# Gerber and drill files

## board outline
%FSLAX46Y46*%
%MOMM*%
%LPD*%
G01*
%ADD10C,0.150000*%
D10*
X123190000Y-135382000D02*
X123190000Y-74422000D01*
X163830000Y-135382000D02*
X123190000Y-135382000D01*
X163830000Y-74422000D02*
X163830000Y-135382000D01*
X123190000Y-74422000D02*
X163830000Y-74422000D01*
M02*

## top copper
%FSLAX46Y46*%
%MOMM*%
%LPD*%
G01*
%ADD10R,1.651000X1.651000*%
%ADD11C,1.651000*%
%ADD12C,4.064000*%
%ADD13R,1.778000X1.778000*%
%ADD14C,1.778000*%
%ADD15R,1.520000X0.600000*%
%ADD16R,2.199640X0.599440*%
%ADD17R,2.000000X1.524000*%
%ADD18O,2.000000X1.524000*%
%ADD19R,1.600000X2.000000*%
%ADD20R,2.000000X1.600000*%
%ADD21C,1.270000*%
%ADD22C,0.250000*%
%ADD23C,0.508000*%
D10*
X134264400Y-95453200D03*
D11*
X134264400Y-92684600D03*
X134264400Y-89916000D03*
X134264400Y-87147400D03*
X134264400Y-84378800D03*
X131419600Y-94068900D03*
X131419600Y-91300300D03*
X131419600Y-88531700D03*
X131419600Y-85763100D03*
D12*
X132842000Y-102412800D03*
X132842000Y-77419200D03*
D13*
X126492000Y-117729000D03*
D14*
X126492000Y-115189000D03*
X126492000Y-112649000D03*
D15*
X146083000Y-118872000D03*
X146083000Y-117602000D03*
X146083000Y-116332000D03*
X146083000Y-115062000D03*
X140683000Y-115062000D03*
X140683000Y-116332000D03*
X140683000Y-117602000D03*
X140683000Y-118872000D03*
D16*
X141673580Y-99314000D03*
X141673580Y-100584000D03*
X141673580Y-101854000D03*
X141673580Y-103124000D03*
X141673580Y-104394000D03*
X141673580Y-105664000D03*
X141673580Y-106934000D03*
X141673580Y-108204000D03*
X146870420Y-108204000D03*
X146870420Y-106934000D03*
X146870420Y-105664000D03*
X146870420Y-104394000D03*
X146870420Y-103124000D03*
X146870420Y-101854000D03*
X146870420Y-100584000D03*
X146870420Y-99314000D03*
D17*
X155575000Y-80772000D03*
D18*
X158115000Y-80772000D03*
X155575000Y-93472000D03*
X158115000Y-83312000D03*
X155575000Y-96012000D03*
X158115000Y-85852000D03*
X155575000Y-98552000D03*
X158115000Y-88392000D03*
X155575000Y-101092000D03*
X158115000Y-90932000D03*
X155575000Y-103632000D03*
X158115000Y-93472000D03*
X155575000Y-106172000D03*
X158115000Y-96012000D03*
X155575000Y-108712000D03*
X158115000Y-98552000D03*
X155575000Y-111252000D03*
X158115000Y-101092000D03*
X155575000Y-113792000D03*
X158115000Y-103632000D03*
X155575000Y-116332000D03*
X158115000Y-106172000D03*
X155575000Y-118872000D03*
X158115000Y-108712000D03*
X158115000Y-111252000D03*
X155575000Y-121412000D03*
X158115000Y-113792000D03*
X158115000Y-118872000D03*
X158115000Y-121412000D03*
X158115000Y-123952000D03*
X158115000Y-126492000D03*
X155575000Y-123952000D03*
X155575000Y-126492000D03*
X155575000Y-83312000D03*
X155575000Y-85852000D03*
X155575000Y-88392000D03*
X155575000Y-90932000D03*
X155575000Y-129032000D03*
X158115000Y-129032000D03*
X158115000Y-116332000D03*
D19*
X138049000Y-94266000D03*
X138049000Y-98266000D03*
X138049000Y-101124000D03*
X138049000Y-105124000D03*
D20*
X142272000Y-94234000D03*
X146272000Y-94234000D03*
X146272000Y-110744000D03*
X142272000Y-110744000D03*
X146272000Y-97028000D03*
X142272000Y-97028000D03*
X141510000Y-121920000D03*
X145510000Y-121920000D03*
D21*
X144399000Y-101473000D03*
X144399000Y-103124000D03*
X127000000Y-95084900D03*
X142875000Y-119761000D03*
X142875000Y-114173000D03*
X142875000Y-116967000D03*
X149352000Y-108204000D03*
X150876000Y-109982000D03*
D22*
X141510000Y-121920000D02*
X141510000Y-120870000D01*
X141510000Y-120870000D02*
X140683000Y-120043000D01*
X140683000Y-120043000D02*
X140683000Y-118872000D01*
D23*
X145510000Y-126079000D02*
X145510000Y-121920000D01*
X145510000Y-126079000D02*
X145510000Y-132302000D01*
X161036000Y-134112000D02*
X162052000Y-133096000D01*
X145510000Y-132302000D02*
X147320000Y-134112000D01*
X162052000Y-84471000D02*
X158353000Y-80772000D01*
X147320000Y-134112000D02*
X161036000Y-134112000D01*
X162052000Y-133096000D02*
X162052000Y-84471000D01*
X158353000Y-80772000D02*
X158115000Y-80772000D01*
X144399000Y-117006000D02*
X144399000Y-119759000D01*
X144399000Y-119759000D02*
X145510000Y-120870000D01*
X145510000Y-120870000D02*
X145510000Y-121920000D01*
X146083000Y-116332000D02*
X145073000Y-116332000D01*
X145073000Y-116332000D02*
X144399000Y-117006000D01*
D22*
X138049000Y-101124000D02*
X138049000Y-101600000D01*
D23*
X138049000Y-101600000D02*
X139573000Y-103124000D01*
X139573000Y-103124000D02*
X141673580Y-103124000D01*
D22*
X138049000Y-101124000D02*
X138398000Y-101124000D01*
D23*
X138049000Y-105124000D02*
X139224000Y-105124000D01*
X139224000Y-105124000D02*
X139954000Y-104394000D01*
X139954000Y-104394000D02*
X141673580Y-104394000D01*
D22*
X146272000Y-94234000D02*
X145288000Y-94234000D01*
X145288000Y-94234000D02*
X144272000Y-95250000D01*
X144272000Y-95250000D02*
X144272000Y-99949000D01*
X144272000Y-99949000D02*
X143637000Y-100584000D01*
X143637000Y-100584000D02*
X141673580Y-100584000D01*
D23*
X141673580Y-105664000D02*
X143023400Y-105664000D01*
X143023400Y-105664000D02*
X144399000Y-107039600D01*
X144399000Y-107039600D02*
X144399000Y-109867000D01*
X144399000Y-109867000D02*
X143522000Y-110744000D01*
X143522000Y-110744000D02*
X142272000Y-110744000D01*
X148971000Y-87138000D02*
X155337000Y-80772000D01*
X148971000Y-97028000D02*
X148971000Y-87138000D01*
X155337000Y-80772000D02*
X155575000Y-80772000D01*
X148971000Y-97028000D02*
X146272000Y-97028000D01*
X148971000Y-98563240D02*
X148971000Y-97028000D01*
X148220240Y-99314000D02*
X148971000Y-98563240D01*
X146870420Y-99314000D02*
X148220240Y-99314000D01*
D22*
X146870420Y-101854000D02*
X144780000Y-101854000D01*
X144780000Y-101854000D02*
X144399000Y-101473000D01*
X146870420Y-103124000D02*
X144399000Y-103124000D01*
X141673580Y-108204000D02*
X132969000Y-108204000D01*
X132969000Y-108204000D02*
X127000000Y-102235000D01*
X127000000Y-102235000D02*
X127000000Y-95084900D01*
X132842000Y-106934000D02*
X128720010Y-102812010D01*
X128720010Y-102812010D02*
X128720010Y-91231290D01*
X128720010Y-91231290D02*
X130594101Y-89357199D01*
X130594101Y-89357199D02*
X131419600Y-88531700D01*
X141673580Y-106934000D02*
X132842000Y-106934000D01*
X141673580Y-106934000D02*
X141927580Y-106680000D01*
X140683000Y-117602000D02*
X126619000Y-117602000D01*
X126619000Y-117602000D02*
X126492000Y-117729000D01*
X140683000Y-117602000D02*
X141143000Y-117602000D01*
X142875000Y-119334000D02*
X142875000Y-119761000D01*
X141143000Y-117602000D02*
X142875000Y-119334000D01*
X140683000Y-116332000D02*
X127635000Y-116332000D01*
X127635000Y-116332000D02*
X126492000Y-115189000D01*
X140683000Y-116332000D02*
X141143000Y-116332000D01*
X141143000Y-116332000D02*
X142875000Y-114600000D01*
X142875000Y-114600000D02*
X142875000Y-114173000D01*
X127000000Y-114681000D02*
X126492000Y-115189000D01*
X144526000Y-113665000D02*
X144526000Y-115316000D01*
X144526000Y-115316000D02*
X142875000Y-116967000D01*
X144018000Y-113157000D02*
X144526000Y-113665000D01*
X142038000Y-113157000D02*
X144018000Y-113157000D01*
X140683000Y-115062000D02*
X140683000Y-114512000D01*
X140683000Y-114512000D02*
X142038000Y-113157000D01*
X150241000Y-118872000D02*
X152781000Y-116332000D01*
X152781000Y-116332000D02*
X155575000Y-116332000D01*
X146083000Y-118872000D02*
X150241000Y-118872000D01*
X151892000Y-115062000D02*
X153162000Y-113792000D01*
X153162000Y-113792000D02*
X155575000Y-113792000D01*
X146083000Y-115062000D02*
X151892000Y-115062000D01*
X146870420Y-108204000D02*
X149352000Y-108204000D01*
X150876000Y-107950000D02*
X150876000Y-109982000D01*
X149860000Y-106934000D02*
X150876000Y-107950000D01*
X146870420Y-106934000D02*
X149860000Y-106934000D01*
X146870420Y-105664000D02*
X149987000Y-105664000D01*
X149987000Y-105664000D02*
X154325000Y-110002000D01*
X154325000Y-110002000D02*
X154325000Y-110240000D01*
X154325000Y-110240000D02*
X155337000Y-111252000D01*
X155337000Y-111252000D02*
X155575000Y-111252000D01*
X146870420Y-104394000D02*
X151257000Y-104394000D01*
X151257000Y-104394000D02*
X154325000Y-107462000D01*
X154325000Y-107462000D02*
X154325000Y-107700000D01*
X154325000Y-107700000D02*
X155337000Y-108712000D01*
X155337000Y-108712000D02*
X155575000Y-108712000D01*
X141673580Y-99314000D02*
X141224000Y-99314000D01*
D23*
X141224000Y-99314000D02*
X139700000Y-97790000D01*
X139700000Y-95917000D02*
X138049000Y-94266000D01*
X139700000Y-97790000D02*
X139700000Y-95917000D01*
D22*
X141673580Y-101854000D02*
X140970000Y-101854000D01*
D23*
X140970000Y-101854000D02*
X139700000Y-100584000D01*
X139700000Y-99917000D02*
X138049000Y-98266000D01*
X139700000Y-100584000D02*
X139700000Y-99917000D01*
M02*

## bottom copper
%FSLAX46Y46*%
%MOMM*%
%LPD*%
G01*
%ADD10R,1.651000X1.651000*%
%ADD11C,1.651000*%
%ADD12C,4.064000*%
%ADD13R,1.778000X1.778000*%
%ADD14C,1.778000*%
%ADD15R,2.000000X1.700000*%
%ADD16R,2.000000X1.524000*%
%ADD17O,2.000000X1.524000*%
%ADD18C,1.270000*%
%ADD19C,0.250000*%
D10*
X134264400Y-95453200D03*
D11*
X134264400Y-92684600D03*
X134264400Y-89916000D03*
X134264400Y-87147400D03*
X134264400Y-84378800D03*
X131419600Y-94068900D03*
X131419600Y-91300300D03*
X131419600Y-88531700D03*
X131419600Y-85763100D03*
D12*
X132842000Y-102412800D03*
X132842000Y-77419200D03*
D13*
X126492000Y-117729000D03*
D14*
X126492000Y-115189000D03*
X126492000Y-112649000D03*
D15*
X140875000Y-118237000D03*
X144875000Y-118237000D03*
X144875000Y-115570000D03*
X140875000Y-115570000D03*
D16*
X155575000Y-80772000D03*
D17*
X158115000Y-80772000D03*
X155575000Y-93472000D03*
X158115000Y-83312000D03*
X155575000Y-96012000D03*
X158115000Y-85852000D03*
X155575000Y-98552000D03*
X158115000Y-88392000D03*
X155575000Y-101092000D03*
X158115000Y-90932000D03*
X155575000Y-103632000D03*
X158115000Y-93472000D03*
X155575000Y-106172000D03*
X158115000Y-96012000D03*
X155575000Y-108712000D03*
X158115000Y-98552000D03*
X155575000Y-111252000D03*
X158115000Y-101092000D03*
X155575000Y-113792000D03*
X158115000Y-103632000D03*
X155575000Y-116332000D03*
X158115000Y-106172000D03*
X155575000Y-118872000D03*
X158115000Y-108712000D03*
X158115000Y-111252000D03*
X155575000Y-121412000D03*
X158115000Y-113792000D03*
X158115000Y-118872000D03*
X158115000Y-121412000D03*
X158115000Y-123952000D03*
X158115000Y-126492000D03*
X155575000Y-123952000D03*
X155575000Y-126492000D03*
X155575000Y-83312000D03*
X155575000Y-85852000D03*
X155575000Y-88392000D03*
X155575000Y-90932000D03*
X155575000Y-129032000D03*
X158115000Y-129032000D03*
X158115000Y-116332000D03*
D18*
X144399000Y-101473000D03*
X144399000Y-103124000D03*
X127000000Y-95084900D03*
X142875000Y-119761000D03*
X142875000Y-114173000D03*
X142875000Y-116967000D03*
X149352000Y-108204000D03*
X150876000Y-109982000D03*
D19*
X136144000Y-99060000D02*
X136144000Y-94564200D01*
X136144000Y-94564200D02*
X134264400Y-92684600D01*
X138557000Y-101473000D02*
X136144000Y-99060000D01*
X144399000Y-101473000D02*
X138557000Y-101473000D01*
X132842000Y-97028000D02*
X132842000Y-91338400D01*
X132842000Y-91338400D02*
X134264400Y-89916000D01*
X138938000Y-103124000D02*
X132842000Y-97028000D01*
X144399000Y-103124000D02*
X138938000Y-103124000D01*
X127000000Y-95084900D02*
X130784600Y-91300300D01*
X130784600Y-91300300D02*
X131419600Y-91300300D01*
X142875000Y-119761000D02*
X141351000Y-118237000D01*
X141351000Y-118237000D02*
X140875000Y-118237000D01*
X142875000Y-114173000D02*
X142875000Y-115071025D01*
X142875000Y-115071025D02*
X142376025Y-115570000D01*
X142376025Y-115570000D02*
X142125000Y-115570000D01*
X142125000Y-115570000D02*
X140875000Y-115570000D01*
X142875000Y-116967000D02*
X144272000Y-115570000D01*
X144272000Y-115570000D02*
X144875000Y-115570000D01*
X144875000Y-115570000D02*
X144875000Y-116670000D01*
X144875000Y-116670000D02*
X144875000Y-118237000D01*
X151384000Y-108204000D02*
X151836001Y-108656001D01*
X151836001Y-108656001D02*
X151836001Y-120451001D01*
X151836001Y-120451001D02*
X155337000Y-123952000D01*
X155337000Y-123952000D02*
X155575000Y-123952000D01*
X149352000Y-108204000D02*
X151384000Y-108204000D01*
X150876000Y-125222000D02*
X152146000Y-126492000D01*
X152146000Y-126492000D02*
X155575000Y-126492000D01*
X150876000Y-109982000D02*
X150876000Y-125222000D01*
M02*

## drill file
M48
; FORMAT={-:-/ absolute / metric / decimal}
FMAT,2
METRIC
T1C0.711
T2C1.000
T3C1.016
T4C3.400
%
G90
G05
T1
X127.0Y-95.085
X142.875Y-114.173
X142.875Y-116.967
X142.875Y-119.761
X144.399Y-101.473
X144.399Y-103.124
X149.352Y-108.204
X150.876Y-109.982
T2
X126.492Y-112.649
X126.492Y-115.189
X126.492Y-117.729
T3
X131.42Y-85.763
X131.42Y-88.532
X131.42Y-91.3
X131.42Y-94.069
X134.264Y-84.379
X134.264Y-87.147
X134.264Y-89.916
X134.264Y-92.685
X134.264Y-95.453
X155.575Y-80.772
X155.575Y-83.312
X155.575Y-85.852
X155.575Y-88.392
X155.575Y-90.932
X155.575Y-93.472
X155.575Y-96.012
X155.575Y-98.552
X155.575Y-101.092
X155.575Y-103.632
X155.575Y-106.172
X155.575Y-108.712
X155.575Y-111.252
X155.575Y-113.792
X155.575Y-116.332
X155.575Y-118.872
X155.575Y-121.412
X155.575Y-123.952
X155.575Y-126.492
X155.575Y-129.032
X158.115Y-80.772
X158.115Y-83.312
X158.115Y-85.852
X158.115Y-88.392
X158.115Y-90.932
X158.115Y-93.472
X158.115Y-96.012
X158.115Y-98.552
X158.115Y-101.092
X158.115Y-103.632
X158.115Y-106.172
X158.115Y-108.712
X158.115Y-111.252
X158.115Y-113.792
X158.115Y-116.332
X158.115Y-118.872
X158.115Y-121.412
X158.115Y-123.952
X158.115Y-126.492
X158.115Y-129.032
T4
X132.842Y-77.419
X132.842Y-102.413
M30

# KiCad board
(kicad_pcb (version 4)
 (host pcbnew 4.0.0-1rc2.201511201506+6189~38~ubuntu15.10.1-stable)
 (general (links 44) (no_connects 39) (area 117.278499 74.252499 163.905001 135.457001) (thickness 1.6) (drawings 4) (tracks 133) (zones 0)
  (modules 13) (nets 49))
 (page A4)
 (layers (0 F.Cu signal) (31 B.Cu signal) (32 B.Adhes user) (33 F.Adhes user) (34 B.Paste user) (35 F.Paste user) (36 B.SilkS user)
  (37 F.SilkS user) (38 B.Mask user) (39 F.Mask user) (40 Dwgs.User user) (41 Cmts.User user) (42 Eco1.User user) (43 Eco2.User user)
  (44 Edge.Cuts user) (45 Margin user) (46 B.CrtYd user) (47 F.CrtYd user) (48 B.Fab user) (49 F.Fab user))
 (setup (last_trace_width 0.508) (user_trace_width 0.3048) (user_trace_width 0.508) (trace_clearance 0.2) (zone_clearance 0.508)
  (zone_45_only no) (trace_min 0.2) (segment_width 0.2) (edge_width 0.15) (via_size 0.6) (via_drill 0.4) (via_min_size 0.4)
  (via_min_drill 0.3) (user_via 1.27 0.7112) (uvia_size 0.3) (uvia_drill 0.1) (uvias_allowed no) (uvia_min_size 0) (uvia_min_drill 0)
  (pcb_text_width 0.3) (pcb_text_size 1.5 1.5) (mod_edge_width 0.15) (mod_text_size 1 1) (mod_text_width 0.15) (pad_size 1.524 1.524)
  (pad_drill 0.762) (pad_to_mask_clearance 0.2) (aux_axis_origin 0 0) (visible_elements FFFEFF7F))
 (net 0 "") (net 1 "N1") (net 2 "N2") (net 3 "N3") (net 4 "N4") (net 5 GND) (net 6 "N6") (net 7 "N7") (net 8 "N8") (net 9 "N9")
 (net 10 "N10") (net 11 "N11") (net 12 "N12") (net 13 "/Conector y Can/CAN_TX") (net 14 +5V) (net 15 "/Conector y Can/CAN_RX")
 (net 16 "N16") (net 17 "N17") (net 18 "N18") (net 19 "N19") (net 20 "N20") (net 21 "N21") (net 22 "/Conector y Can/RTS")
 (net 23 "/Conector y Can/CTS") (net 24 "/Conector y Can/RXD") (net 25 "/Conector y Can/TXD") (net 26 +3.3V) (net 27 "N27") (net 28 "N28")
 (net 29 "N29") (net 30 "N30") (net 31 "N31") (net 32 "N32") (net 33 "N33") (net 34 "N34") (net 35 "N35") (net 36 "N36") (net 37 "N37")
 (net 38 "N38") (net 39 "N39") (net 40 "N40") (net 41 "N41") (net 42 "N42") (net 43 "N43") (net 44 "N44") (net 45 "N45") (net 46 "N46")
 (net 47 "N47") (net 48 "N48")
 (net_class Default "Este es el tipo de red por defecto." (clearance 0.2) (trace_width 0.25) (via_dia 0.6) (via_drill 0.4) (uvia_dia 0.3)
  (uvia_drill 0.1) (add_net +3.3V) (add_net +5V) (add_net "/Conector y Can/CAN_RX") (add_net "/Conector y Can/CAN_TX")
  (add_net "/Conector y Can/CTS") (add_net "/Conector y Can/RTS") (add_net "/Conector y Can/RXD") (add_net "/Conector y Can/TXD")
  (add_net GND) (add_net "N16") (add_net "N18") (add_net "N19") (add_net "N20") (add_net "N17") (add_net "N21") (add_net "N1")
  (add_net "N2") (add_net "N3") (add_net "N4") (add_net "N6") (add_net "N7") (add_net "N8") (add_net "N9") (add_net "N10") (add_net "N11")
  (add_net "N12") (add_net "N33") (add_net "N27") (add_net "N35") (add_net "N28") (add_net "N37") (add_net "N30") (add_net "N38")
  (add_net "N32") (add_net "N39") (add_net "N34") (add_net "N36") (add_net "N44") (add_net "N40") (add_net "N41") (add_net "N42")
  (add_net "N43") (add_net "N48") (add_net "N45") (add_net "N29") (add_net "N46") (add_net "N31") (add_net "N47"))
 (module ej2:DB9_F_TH (layer F.Cu) (at 132.842 89.916 90)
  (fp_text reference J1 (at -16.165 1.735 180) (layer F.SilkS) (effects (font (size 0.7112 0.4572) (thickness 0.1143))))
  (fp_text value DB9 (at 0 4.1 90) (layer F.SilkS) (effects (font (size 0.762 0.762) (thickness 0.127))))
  (pad 1 thru_hole rect (at -5.5372 1.4224 90) (size 1.651 1.651) (drill 1.016) (layers *.Cu *.Mask) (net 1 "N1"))
  (pad 2 thru_hole circle (at -2.7686 1.4224 90) (size 1.651 1.651) (drill 1.016) (layers *.Cu *.Mask) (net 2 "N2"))
  (pad 3 thru_hole circle (at 0 1.4224 90) (size 1.651 1.651) (drill 1.016) (layers *.Cu *.Mask) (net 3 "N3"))
  (pad 4 thru_hole circle (at 2.7686 1.4224 90) (size 1.651 1.651) (drill 1.016) (layers *.Cu *.Mask) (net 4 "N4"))
  (pad 5 thru_hole circle (at 5.5372 1.4224 90) (size 1.651 1.651) (drill 1.016) (layers *.Cu *.Mask) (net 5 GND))
  (pad 6 thru_hole circle (at -4.1529 -1.4224 90) (size 1.651 1.651) (drill 1.016) (layers *.Cu *.Mask) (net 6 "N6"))
  (pad 7 thru_hole circle (at -1.3843 -1.4224 90) (size 1.651 1.651) (drill 1.016) (layers *.Cu *.Mask) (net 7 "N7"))
  (pad 8 thru_hole circle (at 1.3843 -1.4224 90) (size 1.651 1.651) (drill 1.016) (layers *.Cu *.Mask) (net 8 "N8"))
  (pad 9 thru_hole circle (at 4.1529 -1.4224 90) (size 1.651 1.651) (drill 1.016) (layers *.Cu *.Mask) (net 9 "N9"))
  (pad 10 thru_hole circle (at -12.4968 0 90) (size 4.064 4.064) (drill 3.4) (layers *.Cu *.Mask))
  (pad 11 thru_hole circle (at 12.4968 0 90) (size 4.064 4.064) (drill 3.4) (layers *.Cu *.Mask)))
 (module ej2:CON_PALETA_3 (layer F.Cu) (at 126.492 115.189 90)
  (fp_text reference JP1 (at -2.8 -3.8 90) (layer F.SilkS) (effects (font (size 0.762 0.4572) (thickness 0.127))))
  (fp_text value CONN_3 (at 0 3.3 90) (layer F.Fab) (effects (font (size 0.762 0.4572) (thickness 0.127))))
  (pad 1 thru_hole rect (at -2.54 0 90) (size 1.778 1.778) (drill 1) (layers *.Cu *.Mask) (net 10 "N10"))
  (pad 2 thru_hole circle (at 0 0 90) (size 1.778 1.778) (drill 1) (layers *.Cu *.Mask) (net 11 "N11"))
  (pad 3 thru_hole circle (at 2.54 0 90) (size 1.778 1.778) (drill 1) (layers *.Cu *.Mask) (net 5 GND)))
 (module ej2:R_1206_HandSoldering (layer B.Cu) (at 142.875 118.237)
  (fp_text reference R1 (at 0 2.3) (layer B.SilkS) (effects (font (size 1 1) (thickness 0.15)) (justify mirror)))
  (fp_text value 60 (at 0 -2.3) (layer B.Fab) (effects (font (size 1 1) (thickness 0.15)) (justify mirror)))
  (pad 1 smd rect (at -2 0) (size 2 1.7) (layers B.Cu B.Paste B.Mask) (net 10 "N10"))
  (pad 2 smd rect (at 2 0) (size 2 1.7) (layers B.Cu B.Paste B.Mask) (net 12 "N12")))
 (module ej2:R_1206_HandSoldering (layer B.Cu) (at 142.875 115.57 180)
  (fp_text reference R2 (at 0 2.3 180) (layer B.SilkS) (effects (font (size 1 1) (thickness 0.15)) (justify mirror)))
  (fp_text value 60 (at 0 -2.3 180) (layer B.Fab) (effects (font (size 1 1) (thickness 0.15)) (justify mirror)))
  (pad 1 smd rect (at -2 0 180) (size 2 1.7) (layers B.Cu B.Paste B.Mask) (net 12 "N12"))
  (pad 2 smd rect (at 2 0 180) (size 2 1.7) (layers B.Cu B.Paste B.Mask) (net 11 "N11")))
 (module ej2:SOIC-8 (layer F.Cu) (at 143.383 116.967 180)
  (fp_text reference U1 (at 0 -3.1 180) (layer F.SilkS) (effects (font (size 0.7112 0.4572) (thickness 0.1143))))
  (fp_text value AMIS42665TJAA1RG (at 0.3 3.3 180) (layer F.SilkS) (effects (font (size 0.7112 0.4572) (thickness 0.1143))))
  (pad 1 smd rect (at -2.7 -1.905 90) (size 0.6 1.52) (layers F.Cu F.Paste F.Mask) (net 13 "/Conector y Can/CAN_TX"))
  (pad 2 smd rect (at -2.7 -0.635 90) (size 0.6 1.52) (layers F.Cu F.Paste F.Mask) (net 5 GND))
  (pad 3 smd rect (at -2.7 0.635 90) (size 0.6 1.52) (layers F.Cu F.Paste F.Mask) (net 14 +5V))
  (pad 4 smd rect (at -2.7 1.905 90) (size 0.6 1.52) (layers F.Cu F.Paste F.Mask) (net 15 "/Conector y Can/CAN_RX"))
  (pad 5 smd rect (at 2.7 1.905 90) (size 0.6 1.52) (layers F.Cu F.Paste F.Mask) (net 12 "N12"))
  (pad 6 smd rect (at 2.7 0.635 90) (size 0.6 1.52) (layers F.Cu F.Paste F.Mask) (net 11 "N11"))
  (pad 7 smd rect (at 2.7 -0.635 90) (size 0.6 1.52) (layers F.Cu F.Paste F.Mask) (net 10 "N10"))
  (pad 8 smd rect (at 2.7 -1.905 90) (size 0.6 1.52) (layers F.Cu F.Paste F.Mask) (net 5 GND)))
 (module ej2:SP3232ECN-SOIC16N (layer F.Cu) (at 144.272 103.759 270)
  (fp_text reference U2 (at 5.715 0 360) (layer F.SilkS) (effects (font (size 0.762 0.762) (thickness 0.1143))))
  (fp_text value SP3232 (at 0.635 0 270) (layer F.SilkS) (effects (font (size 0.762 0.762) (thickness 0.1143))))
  (pad 1 smd rect (at -4.445 2.59842 270) (size 0.59944 2.19964) (layers F.Cu F.Paste F.Mask) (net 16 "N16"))
  (pad 2 smd rect (at -3.175 2.59842 270) (size 0.59944 2.19964) (layers F.Cu F.Paste F.Mask) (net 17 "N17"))
  (pad 3 smd rect (at -1.905 2.59842 270) (size 0.59944 2.19964) (layers F.Cu F.Paste F.Mask) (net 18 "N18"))
  (pad 4 smd rect (at -0.635 2.59842 270) (size 0.59944 2.19964) (layers F.Cu F.Paste F.Mask) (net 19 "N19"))
  (pad 5 smd rect (at 0.635 2.59842 270) (size 0.59944 2.19964) (layers F.Cu F.Paste F.Mask) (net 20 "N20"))
  (pad 6 smd rect (at 1.905 2.59842 270) (size 0.59944 2.19964) (layers F.Cu F.Paste F.Mask) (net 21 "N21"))
  (pad 7 smd rect (at 3.175 2.59842 270) (size 0.59944 2.19964) (layers F.Cu F.Paste F.Mask) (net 8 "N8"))
  (pad 8 smd rect (at 4.445 2.59842 270) (size 0.59944 2.19964) (layers F.Cu F.Paste F.Mask) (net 7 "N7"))
  (pad 9 smd rect (at 4.445 -2.59842 270) (size 0.59944 2.19964) (layers F.Cu F.Paste F.Mask) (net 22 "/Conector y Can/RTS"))
  (pad 10 smd rect (at 3.175 -2.59842 270) (size 0.59944 2.19964) (layers F.Cu F.Paste F.Mask) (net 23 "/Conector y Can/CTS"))
  (pad 11 smd rect (at 1.905 -2.59842 270) (size 0.59944 2.19964) (layers F.Cu F.Paste F.Mask) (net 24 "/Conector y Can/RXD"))
  (pad 12 smd rect (at 0.635 -2.59842 270) (size 0.59944 2.19964) (layers F.Cu F.Paste F.Mask) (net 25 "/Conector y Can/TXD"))
  (pad 13 smd rect (at -0.635 -2.59842 270) (size 0.59944 2.19964) (layers F.Cu F.Paste F.Mask) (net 3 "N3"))
  (pad 14 smd rect (at -1.905 -2.59842 270) (size 0.59944 2.19964) (layers F.Cu F.Paste F.Mask) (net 2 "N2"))
  (pad 15 smd rect (at -3.175 -2.59842 270) (size 0.59944 2.19964) (layers F.Cu F.Paste F.Mask) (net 5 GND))
  (pad 16 smd rect (at -4.445 -2.59842 270) (size 0.59944 2.19964) (layers F.Cu F.Paste F.Mask) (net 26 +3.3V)))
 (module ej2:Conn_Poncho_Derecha (layer F.Cu) (at 155.575 80.772)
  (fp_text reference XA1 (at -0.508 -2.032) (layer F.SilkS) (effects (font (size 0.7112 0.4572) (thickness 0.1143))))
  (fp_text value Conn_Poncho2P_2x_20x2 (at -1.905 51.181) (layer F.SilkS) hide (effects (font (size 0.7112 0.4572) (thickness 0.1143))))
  (pad 1 thru_hole rect (at 0 0 270) (size 1.524 2) (drill 1.016) (layers *.Cu *.Mask) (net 26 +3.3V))
  (pad 2 thru_hole oval (at 2.54 0 270) (size 1.524 2) (drill 1.016) (layers *.Cu *.Mask) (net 14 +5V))
  (pad 11 thru_hole oval (at 0 12.7 270) (size 1.524 2) (drill 1.016) (layers *.Cu *.Mask) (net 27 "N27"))
  (pad 4 thru_hole oval (at 2.54 2.54 270) (size 1.524 2) (drill 1.016) (layers *.Cu *.Mask) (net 5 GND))
  (pad 13 thru_hole oval (at 0 15.24 270) (size 1.524 2) (drill 1.016) (layers *.Cu *.Mask) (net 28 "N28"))
  (pad 6 thru_hole oval (at 2.54 5.08 270) (size 1.524 2) (drill 1.016) (layers *.Cu *.Mask) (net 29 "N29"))
  (pad 15 thru_hole oval (at 0 17.78 270) (size 1.524 2) (drill 1.016) (layers *.Cu *.Mask) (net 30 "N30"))
  (pad 8 thru_hole oval (at 2.54 7.62 270) (size 1.524 2) (drill 1.016) (layers *.Cu *.Mask) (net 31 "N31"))
  (pad 17 thru_hole oval (at 0 20.32 270) (size 1.524 2) (drill 1.016) (layers *.Cu *.Mask) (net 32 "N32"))
  (pad 10 thru_hole oval (at 2.54 10.16 270) (size 1.524 2) (drill 1.016) (layers *.Cu *.Mask) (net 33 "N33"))
  (pad 19 thru_hole oval (at 0 22.86 270) (size 1.524 2) (drill 1.016) (layers *.Cu *.Mask) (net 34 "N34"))
  (pad 12 thru_hole oval (at 2.54 12.7 270) (size 1.524 2) (drill 1.016) (layers *.Cu *.Mask) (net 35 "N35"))
  (pad 21 thru_hole oval (at 0 25.4 270) (size 1.524 2) (drill 1.016) (layers *.Cu *.Mask) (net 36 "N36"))
  (pad 14 thru_hole oval (at 2.54 15.24 270) (size 1.524 2) (drill 1.016) (layers *.Cu *.Mask) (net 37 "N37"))
  (pad 23 thru_hole oval (at 0 27.94 270) (size 1.524 2) (drill 1.016) (layers *.Cu *.Mask) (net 25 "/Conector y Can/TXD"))
  (pad 16 thru_hole oval (at 2.54 17.78 270) (size 1.524 2) (drill 1.016) (layers *.Cu *.Mask) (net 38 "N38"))
  (pad 25 thru_hole oval (at 0 30.48 270) (size 1.524 2) (drill 1.016) (layers *.Cu *.Mask) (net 24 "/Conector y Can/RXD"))
  (pad 18 thru_hole oval (at 2.54 20.32 270) (size 1.524 2) (drill 1.016) (layers *.Cu *.Mask) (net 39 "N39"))
  (pad 27 thru_hole oval (at 0 33.02 270) (size 1.524 2) (drill 1.016) (layers *.Cu *.Mask) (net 15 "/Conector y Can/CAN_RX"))
  (pad 20 thru_hole oval (at 2.54 22.86 270) (size 1.524 2) (drill 1.016) (layers *.Cu *.Mask) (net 5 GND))
  (pad 29 thru_hole oval (at 0 35.56 270) (size 1.524 2) (drill 1.016) (layers *.Cu *.Mask) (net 13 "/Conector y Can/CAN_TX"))
  (pad 22 thru_hole oval (at 2.54 25.4 270) (size 1.524 2) (drill 1.016) (layers *.Cu *.Mask) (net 5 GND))
  (pad 31 thru_hole oval (at 0 38.1 270) (size 1.524 2) (drill 1.016) (layers *.Cu *.Mask) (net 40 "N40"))
  (pad 24 thru_hole oval (at 2.54 27.94 270) (size 1.524 2) (drill 1.016) (layers *.Cu *.Mask) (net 5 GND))
  (pad 26 thru_hole oval (at 2.54 30.48 270) (size 1.524 2) (drill 1.016) (layers *.Cu *.Mask) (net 5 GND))
  (pad 33 thru_hole oval (at 0 40.64 270) (size 1.524 2) (drill 1.016) (layers *.Cu *.Mask) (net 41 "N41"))
  (pad 28 thru_hole oval (at 2.54 33.02 270) (size 1.524 2) (drill 1.016) (layers *.Cu *.Mask) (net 5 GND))
  (pad 32 thru_hole oval (at 2.54 38.1 270) (size 1.524 2) (drill 1.016) (layers *.Cu *.Mask) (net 5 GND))
  (pad 34 thru_hole oval (at 2.54 40.64 270) (size 1.524 2) (drill 1.016) (layers *.Cu *.Mask) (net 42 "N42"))
  (pad 36 thru_hole oval (at 2.54 43.18 270) (size 1.524 2) (drill 1.016) (layers *.Cu *.Mask) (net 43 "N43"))
  (pad 38 thru_hole oval (at 2.54 45.72 270) (size 1.524 2) (drill 1.016) (layers *.Cu *.Mask) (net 5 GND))
  (pad 35 thru_hole oval (at 0 43.18 270) (size 1.524 2) (drill 1.016) (layers *.Cu *.Mask) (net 22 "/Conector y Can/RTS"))
  (pad 37 thru_hole oval (at 0 45.72 270) (size 1.524 2) (drill 1.016) (layers *.Cu *.Mask) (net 23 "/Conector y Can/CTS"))
  (pad 3 thru_hole oval (at 0 2.54 270) (size 1.524 2) (drill 1.016) (layers *.Cu *.Mask) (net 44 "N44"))
  (pad 5 thru_hole oval (at 0 5.08 270) (size 1.524 2) (drill 1.016) (layers *.Cu *.Mask) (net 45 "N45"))
  (pad 7 thru_hole oval (at 0 7.62 270) (size 1.524 2) (drill 1.016) (layers *.Cu *.Mask) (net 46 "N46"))
  (pad 9 thru_hole oval (at 0 10.16 270) (size 1.524 2) (drill 1.016) (layers *.Cu *.Mask) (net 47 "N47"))
  (pad 39 thru_hole oval (at 0 48.26 270) (size 1.524 2) (drill 1.016) (layers *.Cu *.Mask) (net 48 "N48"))
  (pad 40 thru_hole oval (at 2.54 48.26 270) (size 1.524 2) (drill 1.016) (layers *.Cu *.Mask) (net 5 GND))
  (pad 30 thru_hole oval (at 2.54 35.56 270) (size 1.524 2) (drill 1.016) (layers *.Cu *.Mask) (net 5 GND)))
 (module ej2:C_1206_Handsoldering (layer F.Cu) (at 138.049 96.266 270)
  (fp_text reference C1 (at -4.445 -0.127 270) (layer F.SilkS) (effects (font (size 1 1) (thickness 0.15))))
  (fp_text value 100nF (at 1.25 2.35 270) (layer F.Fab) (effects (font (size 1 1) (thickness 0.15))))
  (pad 1 smd rect (at -2 0 270) (size 2 1.6) (layers F.Cu F.Paste F.Mask) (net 16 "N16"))
  (pad 2 smd rect (at 2 0 270) (size 2 1.6) (layers F.Cu F.Paste F.Mask) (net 18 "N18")))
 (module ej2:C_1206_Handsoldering (layer F.Cu) (at 138.049 103.124 270)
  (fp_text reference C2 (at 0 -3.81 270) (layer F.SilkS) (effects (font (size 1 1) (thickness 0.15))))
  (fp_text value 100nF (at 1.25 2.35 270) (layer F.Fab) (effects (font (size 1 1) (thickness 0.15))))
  (pad 1 smd rect (at -2 0 270) (size 2 1.6) (layers F.Cu F.Paste F.Mask) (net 19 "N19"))
  (pad 2 smd rect (at 2 0 270) (size 2 1.6) (layers F.Cu F.Paste F.Mask) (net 20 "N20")))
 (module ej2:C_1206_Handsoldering (layer F.Cu) (at 144.272 94.234)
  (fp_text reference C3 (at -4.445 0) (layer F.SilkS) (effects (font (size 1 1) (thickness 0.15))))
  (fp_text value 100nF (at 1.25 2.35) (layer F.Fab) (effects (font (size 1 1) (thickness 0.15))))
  (pad 1 smd rect (at -2 0) (size 2 1.6) (layers F.Cu F.Paste F.Mask) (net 5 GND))
  (pad 2 smd rect (at 2 0) (size 2 1.6) (layers F.Cu F.Paste F.Mask) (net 17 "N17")))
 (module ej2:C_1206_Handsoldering (layer F.Cu) (at 144.272 110.744 180)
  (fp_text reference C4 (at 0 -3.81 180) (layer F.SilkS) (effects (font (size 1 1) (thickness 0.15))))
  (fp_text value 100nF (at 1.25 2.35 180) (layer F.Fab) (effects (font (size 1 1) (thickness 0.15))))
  (pad 1 smd rect (at -2 0 180) (size 2 1.6) (layers F.Cu F.Paste F.Mask) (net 5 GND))
  (pad 2 smd rect (at 2 0 180) (size 2 1.6) (layers F.Cu F.Paste F.Mask) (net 21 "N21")))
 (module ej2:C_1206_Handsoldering (layer F.Cu) (at 144.272 97.028 180)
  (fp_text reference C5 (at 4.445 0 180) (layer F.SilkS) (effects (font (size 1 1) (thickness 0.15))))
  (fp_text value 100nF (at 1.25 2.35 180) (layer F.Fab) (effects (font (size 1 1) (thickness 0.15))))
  (pad 1 smd rect (at -2 0 180) (size 2 1.6) (layers F.Cu F.Paste F.Mask) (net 26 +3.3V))
  (pad 2 smd rect (at 2 0 180) (size 2 1.6) (layers F.Cu F.Paste F.Mask) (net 5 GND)))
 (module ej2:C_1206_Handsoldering (layer F.Cu) (at 143.51 121.92)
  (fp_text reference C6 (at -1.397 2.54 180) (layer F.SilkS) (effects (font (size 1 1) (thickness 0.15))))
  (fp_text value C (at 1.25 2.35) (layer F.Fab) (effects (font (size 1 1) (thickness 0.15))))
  (pad 1 smd rect (at -2 0) (size 2 1.6) (layers F.Cu F.Paste F.Mask) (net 5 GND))
  (pad 2 smd rect (at 2 0) (size 2 1.6) (layers F.Cu F.Paste F.Mask) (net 14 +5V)))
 (gr_line (start 123.19 135.382) (end 123.19 74.422) (angle 90) (layer Edge.Cuts) (width 0.15))
 (gr_line (start 163.83 135.382) (end 123.19 135.382) (angle 90) (layer Edge.Cuts) (width 0.15))
 (gr_line (start 163.83 74.422) (end 163.83 135.382) (angle 90) (layer Edge.Cuts) (width 0.15))
 (gr_line (start 123.19 74.422) (end 163.83 74.422) (angle 90) (layer Edge.Cuts) (width 0.15))
 (segment (start 141.51 121.92) (end 141.51 120.87) (width 0.25) (layer F.Cu) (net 5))
 (segment (start 141.51 120.87) (end 140.683 120.043) (width 0.25) (layer F.Cu) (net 5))
 (segment (start 140.683 120.043) (end 140.683 118.872) (width 0.25) (layer F.Cu) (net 5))
 (segment (start 145.51 126.079) (end 145.51 121.92) (width 0.508) (layer F.Cu) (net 14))
 (segment (start 145.51 126.079) (end 145.51 132.302) (width 0.508) (layer F.Cu) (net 14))
 (segment (start 161.036 134.112) (end 162.052 133.096) (width 0.508) (layer F.Cu) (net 14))
 (segment (start 145.51 132.302) (end 147.32 134.112) (width 0.508) (layer F.Cu) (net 14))
 (segment (start 162.052 84.471) (end 158.353 80.772) (width 0.508) (layer F.Cu) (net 14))
 (segment (start 147.32 134.112) (end 161.036 134.112) (width 0.508) (layer F.Cu) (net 14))
 (segment (start 162.052 133.096) (end 162.052 84.471) (width 0.508) (layer F.Cu) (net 14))
 (segment (start 158.353 80.772) (end 158.115 80.772) (width 0.508) (layer F.Cu) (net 14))
 (segment (start 144.399 117.006) (end 144.399 119.759) (width 0.508) (layer F.Cu) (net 14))
 (segment (start 144.399 119.759) (end 145.51 120.87) (width 0.508) (layer F.Cu) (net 14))
 (segment (start 145.51 120.87) (end 145.51 121.92) (width 0.508) (layer F.Cu) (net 14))
 (segment (start 146.083 116.332) (end 145.073 116.332) (width 0.508) (layer F.Cu) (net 14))
 (segment (start 145.073 116.332) (end 144.399 117.006) (width 0.508) (layer F.Cu) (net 14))
 (segment (start 138.049 101.124) (end 138.049 101.6) (width 0.25) (layer F.Cu) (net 19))
 (segment (start 138.049 101.6) (end 139.573 103.124) (width 0.508) (layer F.Cu) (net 19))
 (segment (start 139.573 103.124) (end 141.67358 103.124) (width 0.508) (layer F.Cu) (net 19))
 (segment (start 138.049 101.124) (end 138.398 101.124) (width 0.25) (layer F.Cu) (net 19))
 (segment (start 138.049 105.124) (end 139.224 105.124) (width 0.508) (layer F.Cu) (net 20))
 (segment (start 139.224 105.124) (end 139.954 104.394) (width 0.508) (layer F.Cu) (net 20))
 (segment (start 139.954 104.394) (end 141.67358 104.394) (width 0.508) (layer F.Cu) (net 20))
 (segment (start 146.272 94.234) (end 145.288 94.234) (width 0.25) (layer F.Cu) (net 17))
 (segment (start 145.288 94.234) (end 144.272 95.25) (width 0.25) (layer F.Cu) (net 17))
 (segment (start 144.272 95.25) (end 144.272 99.949) (width 0.25) (layer F.Cu) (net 17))
 (segment (start 144.272 99.949) (end 143.637 100.584) (width 0.25) (layer F.Cu) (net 17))
 (segment (start 143.637 100.584) (end 141.67358 100.584) (width 0.25) (layer F.Cu) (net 17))
 (segment (start 141.67358 105.664) (end 143.0234 105.664) (width 0.508) (layer F.Cu) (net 21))
 (segment (start 143.0234 105.664) (end 144.399 107.0396) (width 0.508) (layer F.Cu) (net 21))
 (segment (start 144.399 107.0396) (end 144.399 109.867) (width 0.508) (layer F.Cu) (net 21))
 (segment (start 144.399 109.867) (end 143.522 110.744) (width 0.508) (layer F.Cu) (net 21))
 (segment (start 143.522 110.744) (end 142.272 110.744) (width 0.508) (layer F.Cu) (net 21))
 (segment (start 148.971 87.138) (end 155.337 80.772) (width 0.508) (layer F.Cu) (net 26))
 (segment (start 148.971 97.028) (end 148.971 87.138) (width 0.508) (layer F.Cu) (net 26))
 (segment (start 155.337 80.772) (end 155.575 80.772) (width 0.508) (layer F.Cu) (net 26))
 (segment (start 148.971 97.028) (end 146.272 97.028) (width 0.508) (layer F.Cu) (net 26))
 (segment (start 148.971 98.56324) (end 148.971 97.028) (width 0.508) (layer F.Cu) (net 26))
 (segment (start 148.22024 99.314) (end 148.971 98.56324) (width 0.508) (layer F.Cu) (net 26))
 (segment (start 146.87042 99.314) (end 148.22024 99.314) (width 0.508) (layer F.Cu) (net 26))
 (segment (start 136.144 99.06) (end 136.144 94.5642) (width 0.25) (layer B.Cu) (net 2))
 (segment (start 136.144 94.5642) (end 134.2644 92.6846) (width 0.25) (layer B.Cu) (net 2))
 (segment (start 138.557 101.473) (end 136.144 99.06) (width 0.25) (layer B.Cu) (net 2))
 (segment (start 144.399 101.473) (end 138.557 101.473) (width 0.25) (layer B.Cu) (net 2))
 (segment (start 146.87042 101.854) (end 144.78 101.854) (width 0.25) (layer F.Cu) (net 2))
 (segment (start 144.78 101.854) (end 144.399 101.473) (width 0.25) (layer F.Cu) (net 2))
 (via (at 144.399 101.473) (size 1.27) (drill 0.7112) (layers F.Cu B.Cu) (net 2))
 (segment (start 132.842 97.028) (end 132.842 91.3384) (width 0.25) (layer B.Cu) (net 3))
 (segment (start 132.842 91.3384) (end 134.2644 89.916) (width 0.25) (layer B.Cu) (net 3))
 (segment (start 138.938 103.124) (end 132.842 97.028) (width 0.25) (layer B.Cu) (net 3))
 (segment (start 144.399 103.124) (end 138.938 103.124) (width 0.25) (layer B.Cu) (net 3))
 (segment (start 146.87042 103.124) (end 144.399 103.124) (width 0.25) (layer F.Cu) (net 3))
 (via (at 144.399 103.124) (size 1.27) (drill 0.7112) (layers F.Cu B.Cu) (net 3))
 (segment (start 127 95.0849) (end 130.7846 91.3003) (width 0.25) (layer B.Cu) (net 7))
 (segment (start 130.7846 91.3003) (end 131.4196 91.3003) (width 0.25) (layer B.Cu) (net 7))
 (via (at 127 95.0849) (size 1.27) (drill 0.7112) (layers F.Cu B.Cu) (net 7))
 (segment (start 141.67358 108.204) (end 132.969 108.204) (width 0.25) (layer F.Cu) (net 7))
 (segment (start 132.969 108.204) (end 127 102.235) (width 0.25) (layer F.Cu) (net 7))
 (segment (start 127 102.235) (end 127 95.0849) (width 0.25) (layer F.Cu) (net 7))
 (segment (start 132.842 106.934) (end 128.72001 102.81201) (width 0.25) (layer F.Cu) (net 8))
 (segment (start 128.72001 102.81201) (end 128.72001 91.23129) (width 0.25) (layer F.Cu) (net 8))
 (segment (start 128.72001 91.23129) (end 130.594101 89.357199) (width 0.25) (layer F.Cu) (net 8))
 (segment (start 130.594101 89.357199) (end 131.4196 88.5317) (width 0.25) (layer F.Cu) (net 8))
 (segment (start 141.67358 106.934) (end 132.842 106.934) (width 0.25) (layer F.Cu) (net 8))
 (segment (start 141.67358 106.934) (end 141.92758 106.68) (width 0.25) (layer F.Cu) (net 8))
 (segment (start 140.683 117.602) (end 126.619 117.602) (width 0.25) (layer F.Cu) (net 10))
 (segment (start 126.619 117.602) (end 126.492 117.729) (width 0.25) (layer F.Cu) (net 10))
 (segment (start 142.875 119.761) (end 141.351 118.237) (width 0.25) (layer B.Cu) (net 10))
 (segment (start 141.351 118.237) (end 140.875 118.237) (width 0.25) (layer B.Cu) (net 10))
 (segment (start 140.683 117.602) (end 141.143 117.602) (width 0.25) (layer F.Cu) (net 10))
 (segment (start 142.875 119.334) (end 142.875 119.761) (width 0.25) (layer F.Cu) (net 10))
 (segment (start 141.143 117.602) (end 142.875 119.334) (width 0.25) (layer F.Cu) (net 10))
 (via (at 142.875 119.761) (size 1.27) (drill 0.7112) (layers F.Cu B.Cu) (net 10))
 (segment (start 140.683 116.332) (end 127.635 116.332) (width 0.25) (layer F.Cu) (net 11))
 (segment (start 127.635 116.332) (end 126.492 115.189) (width 0.25) (layer F.Cu) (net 11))
 (segment (start 142.875 114.173) (end 142.875 115.071025) (width 0.25) (layer B.Cu) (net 11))
 (segment (start 142.875 115.071025) (end 142.376025 115.57) (width 0.25) (layer B.Cu) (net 11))
 (segment (start 142.376025 115.57) (end 142.125 115.57) (width 0.25) (layer B.Cu) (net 11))
 (segment (start 142.125 115.57) (end 140.875 115.57) (width 0.25) (layer B.Cu) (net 11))
 (segment (start 140.683 116.332) (end 141.143 116.332) (width 0.25) (layer F.Cu) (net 11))
 (segment (start 141.143 116.332) (end 142.875 114.6) (width 0.25) (layer F.Cu) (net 11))
 (segment (start 142.875 114.6) (end 142.875 114.173) (width 0.25) (layer F.Cu) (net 11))
 (via (at 142.875 114.173) (size 1.27) (drill 0.7112) (layers F.Cu B.Cu) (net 11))
 (segment (start 127 114.681) (end 126.492 115.189) (width 0.25) (layer F.Cu) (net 11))
 (segment (start 142.875 116.967) (end 144.272 115.57) (width 0.25) (layer B.Cu) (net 12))
 (segment (start 144.272 115.57) (end 144.875 115.57) (width 0.25) (layer B.Cu) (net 12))
 (segment (start 144.526 113.665) (end 144.526 115.316) (width 0.25) (layer F.Cu) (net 12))
 (segment (start 144.526 115.316) (end 142.875 116.967) (width 0.25) (layer F.Cu) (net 12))
 (via (at 142.875 116.967) (size 1.27) (drill 0.7112) (layers F.Cu B.Cu) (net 12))
 (segment (start 144.018 113.157) (end 144.526 113.665) (width 0.25) (layer F.Cu) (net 12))
 (segment (start 142.038 113.157) (end 144.018 113.157) (width 0.25) (layer F.Cu) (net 12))
 (segment (start 140.683 115.062) (end 140.683 114.512) (width 0.25) (layer F.Cu) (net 12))
 (segment (start 140.683 114.512) (end 142.038 113.157) (width 0.25) (layer F.Cu) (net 12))
 (segment (start 144.875 115.57) (end 144.875 116.67) (width 0.25) (layer B.Cu) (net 12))
 (segment (start 144.875 116.67) (end 144.875 118.237) (width 0.25) (layer B.Cu) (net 12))
 (segment (start 150.241 118.872) (end 152.781 116.332) (width 0.25) (layer F.Cu) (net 13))
 (segment (start 152.781 116.332) (end 155.575 116.332) (width 0.25) (layer F.Cu) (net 13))
 (segment (start 146.083 118.872) (end 150.241 118.872) (width 0.25) (layer F.Cu) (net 13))
 (segment (start 151.892 115.062) (end 153.162 113.792) (width 0.25) (layer F.Cu) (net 15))
 (segment (start 153.162 113.792) (end 155.575 113.792) (width 0.25) (layer F.Cu) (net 15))
 (segment (start 146.083 115.062) (end 151.892 115.062) (width 0.25) (layer F.Cu) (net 15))
 (segment (start 151.384 108.204) (end 151.836001 108.656001) (width 0.25) (layer B.Cu) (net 22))
 (segment (start 151.836001 108.656001) (end 151.836001 120.451001) (width 0.25) (layer B.Cu) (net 22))
 (segment (start 151.836001 120.451001) (end 155.337 123.952) (width 0.25) (layer B.Cu) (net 22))
 (segment (start 155.337 123.952) (end 155.575 123.952) (width 0.25) (layer B.Cu) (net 22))
 (segment (start 149.352 108.204) (end 151.384 108.204) (width 0.25) (layer B.Cu) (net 22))
 (via (at 149.352 108.204) (size 1.27) (drill 0.7112) (layers F.Cu B.Cu) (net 22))
 (segment (start 146.87042 108.204) (end 149.352 108.204) (width 0.25) (layer F.Cu) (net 22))
 (segment (start 150.876 125.222) (end 152.146 126.492) (width 0.25) (layer B.Cu) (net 23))
 (segment (start 152.146 126.492) (end 155.575 126.492) (width 0.25) (layer B.Cu) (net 23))
 (segment (start 150.876 109.982) (end 150.876 125.222) (width 0.25) (layer B.Cu) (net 23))
 (segment (start 150.876 107.95) (end 150.876 109.982) (width 0.25) (layer F.Cu) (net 23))
 (via (at 150.876 109.982) (size 1.27) (drill 0.7112) (layers F.Cu B.Cu) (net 23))
 (segment (start 149.86 106.934) (end 150.876 107.95) (width 0.25) (layer F.Cu) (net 23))
 (segment (start 146.87042 106.934) (end 149.86 106.934) (width 0.25) (layer F.Cu) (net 23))
 (segment (start 146.87042 105.664) (end 149.987 105.664) (width 0.25) (layer F.Cu) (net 24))
 (segment (start 149.987 105.664) (end 154.325 110.002) (width 0.25) (layer F.Cu) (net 24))
 (segment (start 154.325 110.002) (end 154.325 110.24) (width 0.25) (layer F.Cu) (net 24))
 (segment (start 154.325 110.24) (end 155.337 111.252) (width 0.25) (layer F.Cu) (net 24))
 (segment (start 155.337 111.252) (end 155.575 111.252) (width 0.25) (layer F.Cu) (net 24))
 (segment (start 146.87042 104.394) (end 151.257 104.394) (width 0.25) (layer F.Cu) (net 25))
 (segment (start 151.257 104.394) (end 154.325 107.462) (width 0.25) (layer F.Cu) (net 25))
 (segment (start 154.325 107.462) (end 154.325 107.7) (width 0.25) (layer F.Cu) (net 25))
 (segment (start 154.325 107.7) (end 155.337 108.712) (width 0.25) (layer F.Cu) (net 25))
 (segment (start 155.337 108.712) (end 155.575 108.712) (width 0.25) (layer F.Cu) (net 25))
 (segment (start 141.67358 99.314) (end 141.224 99.314) (width 0.25) (layer F.Cu) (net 16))
 (segment (start 141.224 99.314) (end 139.7 97.79) (width 0.508) (layer F.Cu) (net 16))
 (segment (start 139.7 95.917) (end 138.049 94.266) (width 0.508) (layer F.Cu) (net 16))
 (segment (start 139.7 97.79) (end 139.7 95.917) (width 0.508) (layer F.Cu) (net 16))
 (segment (start 141.67358 101.854) (end 140.97 101.854) (width 0.25) (layer F.Cu) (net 18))
 (segment (start 140.97 101.854) (end 139.7 100.584) (width 0.508) (layer F.Cu) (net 18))
 (segment (start 139.7 99.917) (end 138.049 98.266) (width 0.508) (layer F.Cu) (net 18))
 (segment (start 139.7 100.584) (end 139.7 99.917) (width 0.508) (layer F.Cu) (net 18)))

